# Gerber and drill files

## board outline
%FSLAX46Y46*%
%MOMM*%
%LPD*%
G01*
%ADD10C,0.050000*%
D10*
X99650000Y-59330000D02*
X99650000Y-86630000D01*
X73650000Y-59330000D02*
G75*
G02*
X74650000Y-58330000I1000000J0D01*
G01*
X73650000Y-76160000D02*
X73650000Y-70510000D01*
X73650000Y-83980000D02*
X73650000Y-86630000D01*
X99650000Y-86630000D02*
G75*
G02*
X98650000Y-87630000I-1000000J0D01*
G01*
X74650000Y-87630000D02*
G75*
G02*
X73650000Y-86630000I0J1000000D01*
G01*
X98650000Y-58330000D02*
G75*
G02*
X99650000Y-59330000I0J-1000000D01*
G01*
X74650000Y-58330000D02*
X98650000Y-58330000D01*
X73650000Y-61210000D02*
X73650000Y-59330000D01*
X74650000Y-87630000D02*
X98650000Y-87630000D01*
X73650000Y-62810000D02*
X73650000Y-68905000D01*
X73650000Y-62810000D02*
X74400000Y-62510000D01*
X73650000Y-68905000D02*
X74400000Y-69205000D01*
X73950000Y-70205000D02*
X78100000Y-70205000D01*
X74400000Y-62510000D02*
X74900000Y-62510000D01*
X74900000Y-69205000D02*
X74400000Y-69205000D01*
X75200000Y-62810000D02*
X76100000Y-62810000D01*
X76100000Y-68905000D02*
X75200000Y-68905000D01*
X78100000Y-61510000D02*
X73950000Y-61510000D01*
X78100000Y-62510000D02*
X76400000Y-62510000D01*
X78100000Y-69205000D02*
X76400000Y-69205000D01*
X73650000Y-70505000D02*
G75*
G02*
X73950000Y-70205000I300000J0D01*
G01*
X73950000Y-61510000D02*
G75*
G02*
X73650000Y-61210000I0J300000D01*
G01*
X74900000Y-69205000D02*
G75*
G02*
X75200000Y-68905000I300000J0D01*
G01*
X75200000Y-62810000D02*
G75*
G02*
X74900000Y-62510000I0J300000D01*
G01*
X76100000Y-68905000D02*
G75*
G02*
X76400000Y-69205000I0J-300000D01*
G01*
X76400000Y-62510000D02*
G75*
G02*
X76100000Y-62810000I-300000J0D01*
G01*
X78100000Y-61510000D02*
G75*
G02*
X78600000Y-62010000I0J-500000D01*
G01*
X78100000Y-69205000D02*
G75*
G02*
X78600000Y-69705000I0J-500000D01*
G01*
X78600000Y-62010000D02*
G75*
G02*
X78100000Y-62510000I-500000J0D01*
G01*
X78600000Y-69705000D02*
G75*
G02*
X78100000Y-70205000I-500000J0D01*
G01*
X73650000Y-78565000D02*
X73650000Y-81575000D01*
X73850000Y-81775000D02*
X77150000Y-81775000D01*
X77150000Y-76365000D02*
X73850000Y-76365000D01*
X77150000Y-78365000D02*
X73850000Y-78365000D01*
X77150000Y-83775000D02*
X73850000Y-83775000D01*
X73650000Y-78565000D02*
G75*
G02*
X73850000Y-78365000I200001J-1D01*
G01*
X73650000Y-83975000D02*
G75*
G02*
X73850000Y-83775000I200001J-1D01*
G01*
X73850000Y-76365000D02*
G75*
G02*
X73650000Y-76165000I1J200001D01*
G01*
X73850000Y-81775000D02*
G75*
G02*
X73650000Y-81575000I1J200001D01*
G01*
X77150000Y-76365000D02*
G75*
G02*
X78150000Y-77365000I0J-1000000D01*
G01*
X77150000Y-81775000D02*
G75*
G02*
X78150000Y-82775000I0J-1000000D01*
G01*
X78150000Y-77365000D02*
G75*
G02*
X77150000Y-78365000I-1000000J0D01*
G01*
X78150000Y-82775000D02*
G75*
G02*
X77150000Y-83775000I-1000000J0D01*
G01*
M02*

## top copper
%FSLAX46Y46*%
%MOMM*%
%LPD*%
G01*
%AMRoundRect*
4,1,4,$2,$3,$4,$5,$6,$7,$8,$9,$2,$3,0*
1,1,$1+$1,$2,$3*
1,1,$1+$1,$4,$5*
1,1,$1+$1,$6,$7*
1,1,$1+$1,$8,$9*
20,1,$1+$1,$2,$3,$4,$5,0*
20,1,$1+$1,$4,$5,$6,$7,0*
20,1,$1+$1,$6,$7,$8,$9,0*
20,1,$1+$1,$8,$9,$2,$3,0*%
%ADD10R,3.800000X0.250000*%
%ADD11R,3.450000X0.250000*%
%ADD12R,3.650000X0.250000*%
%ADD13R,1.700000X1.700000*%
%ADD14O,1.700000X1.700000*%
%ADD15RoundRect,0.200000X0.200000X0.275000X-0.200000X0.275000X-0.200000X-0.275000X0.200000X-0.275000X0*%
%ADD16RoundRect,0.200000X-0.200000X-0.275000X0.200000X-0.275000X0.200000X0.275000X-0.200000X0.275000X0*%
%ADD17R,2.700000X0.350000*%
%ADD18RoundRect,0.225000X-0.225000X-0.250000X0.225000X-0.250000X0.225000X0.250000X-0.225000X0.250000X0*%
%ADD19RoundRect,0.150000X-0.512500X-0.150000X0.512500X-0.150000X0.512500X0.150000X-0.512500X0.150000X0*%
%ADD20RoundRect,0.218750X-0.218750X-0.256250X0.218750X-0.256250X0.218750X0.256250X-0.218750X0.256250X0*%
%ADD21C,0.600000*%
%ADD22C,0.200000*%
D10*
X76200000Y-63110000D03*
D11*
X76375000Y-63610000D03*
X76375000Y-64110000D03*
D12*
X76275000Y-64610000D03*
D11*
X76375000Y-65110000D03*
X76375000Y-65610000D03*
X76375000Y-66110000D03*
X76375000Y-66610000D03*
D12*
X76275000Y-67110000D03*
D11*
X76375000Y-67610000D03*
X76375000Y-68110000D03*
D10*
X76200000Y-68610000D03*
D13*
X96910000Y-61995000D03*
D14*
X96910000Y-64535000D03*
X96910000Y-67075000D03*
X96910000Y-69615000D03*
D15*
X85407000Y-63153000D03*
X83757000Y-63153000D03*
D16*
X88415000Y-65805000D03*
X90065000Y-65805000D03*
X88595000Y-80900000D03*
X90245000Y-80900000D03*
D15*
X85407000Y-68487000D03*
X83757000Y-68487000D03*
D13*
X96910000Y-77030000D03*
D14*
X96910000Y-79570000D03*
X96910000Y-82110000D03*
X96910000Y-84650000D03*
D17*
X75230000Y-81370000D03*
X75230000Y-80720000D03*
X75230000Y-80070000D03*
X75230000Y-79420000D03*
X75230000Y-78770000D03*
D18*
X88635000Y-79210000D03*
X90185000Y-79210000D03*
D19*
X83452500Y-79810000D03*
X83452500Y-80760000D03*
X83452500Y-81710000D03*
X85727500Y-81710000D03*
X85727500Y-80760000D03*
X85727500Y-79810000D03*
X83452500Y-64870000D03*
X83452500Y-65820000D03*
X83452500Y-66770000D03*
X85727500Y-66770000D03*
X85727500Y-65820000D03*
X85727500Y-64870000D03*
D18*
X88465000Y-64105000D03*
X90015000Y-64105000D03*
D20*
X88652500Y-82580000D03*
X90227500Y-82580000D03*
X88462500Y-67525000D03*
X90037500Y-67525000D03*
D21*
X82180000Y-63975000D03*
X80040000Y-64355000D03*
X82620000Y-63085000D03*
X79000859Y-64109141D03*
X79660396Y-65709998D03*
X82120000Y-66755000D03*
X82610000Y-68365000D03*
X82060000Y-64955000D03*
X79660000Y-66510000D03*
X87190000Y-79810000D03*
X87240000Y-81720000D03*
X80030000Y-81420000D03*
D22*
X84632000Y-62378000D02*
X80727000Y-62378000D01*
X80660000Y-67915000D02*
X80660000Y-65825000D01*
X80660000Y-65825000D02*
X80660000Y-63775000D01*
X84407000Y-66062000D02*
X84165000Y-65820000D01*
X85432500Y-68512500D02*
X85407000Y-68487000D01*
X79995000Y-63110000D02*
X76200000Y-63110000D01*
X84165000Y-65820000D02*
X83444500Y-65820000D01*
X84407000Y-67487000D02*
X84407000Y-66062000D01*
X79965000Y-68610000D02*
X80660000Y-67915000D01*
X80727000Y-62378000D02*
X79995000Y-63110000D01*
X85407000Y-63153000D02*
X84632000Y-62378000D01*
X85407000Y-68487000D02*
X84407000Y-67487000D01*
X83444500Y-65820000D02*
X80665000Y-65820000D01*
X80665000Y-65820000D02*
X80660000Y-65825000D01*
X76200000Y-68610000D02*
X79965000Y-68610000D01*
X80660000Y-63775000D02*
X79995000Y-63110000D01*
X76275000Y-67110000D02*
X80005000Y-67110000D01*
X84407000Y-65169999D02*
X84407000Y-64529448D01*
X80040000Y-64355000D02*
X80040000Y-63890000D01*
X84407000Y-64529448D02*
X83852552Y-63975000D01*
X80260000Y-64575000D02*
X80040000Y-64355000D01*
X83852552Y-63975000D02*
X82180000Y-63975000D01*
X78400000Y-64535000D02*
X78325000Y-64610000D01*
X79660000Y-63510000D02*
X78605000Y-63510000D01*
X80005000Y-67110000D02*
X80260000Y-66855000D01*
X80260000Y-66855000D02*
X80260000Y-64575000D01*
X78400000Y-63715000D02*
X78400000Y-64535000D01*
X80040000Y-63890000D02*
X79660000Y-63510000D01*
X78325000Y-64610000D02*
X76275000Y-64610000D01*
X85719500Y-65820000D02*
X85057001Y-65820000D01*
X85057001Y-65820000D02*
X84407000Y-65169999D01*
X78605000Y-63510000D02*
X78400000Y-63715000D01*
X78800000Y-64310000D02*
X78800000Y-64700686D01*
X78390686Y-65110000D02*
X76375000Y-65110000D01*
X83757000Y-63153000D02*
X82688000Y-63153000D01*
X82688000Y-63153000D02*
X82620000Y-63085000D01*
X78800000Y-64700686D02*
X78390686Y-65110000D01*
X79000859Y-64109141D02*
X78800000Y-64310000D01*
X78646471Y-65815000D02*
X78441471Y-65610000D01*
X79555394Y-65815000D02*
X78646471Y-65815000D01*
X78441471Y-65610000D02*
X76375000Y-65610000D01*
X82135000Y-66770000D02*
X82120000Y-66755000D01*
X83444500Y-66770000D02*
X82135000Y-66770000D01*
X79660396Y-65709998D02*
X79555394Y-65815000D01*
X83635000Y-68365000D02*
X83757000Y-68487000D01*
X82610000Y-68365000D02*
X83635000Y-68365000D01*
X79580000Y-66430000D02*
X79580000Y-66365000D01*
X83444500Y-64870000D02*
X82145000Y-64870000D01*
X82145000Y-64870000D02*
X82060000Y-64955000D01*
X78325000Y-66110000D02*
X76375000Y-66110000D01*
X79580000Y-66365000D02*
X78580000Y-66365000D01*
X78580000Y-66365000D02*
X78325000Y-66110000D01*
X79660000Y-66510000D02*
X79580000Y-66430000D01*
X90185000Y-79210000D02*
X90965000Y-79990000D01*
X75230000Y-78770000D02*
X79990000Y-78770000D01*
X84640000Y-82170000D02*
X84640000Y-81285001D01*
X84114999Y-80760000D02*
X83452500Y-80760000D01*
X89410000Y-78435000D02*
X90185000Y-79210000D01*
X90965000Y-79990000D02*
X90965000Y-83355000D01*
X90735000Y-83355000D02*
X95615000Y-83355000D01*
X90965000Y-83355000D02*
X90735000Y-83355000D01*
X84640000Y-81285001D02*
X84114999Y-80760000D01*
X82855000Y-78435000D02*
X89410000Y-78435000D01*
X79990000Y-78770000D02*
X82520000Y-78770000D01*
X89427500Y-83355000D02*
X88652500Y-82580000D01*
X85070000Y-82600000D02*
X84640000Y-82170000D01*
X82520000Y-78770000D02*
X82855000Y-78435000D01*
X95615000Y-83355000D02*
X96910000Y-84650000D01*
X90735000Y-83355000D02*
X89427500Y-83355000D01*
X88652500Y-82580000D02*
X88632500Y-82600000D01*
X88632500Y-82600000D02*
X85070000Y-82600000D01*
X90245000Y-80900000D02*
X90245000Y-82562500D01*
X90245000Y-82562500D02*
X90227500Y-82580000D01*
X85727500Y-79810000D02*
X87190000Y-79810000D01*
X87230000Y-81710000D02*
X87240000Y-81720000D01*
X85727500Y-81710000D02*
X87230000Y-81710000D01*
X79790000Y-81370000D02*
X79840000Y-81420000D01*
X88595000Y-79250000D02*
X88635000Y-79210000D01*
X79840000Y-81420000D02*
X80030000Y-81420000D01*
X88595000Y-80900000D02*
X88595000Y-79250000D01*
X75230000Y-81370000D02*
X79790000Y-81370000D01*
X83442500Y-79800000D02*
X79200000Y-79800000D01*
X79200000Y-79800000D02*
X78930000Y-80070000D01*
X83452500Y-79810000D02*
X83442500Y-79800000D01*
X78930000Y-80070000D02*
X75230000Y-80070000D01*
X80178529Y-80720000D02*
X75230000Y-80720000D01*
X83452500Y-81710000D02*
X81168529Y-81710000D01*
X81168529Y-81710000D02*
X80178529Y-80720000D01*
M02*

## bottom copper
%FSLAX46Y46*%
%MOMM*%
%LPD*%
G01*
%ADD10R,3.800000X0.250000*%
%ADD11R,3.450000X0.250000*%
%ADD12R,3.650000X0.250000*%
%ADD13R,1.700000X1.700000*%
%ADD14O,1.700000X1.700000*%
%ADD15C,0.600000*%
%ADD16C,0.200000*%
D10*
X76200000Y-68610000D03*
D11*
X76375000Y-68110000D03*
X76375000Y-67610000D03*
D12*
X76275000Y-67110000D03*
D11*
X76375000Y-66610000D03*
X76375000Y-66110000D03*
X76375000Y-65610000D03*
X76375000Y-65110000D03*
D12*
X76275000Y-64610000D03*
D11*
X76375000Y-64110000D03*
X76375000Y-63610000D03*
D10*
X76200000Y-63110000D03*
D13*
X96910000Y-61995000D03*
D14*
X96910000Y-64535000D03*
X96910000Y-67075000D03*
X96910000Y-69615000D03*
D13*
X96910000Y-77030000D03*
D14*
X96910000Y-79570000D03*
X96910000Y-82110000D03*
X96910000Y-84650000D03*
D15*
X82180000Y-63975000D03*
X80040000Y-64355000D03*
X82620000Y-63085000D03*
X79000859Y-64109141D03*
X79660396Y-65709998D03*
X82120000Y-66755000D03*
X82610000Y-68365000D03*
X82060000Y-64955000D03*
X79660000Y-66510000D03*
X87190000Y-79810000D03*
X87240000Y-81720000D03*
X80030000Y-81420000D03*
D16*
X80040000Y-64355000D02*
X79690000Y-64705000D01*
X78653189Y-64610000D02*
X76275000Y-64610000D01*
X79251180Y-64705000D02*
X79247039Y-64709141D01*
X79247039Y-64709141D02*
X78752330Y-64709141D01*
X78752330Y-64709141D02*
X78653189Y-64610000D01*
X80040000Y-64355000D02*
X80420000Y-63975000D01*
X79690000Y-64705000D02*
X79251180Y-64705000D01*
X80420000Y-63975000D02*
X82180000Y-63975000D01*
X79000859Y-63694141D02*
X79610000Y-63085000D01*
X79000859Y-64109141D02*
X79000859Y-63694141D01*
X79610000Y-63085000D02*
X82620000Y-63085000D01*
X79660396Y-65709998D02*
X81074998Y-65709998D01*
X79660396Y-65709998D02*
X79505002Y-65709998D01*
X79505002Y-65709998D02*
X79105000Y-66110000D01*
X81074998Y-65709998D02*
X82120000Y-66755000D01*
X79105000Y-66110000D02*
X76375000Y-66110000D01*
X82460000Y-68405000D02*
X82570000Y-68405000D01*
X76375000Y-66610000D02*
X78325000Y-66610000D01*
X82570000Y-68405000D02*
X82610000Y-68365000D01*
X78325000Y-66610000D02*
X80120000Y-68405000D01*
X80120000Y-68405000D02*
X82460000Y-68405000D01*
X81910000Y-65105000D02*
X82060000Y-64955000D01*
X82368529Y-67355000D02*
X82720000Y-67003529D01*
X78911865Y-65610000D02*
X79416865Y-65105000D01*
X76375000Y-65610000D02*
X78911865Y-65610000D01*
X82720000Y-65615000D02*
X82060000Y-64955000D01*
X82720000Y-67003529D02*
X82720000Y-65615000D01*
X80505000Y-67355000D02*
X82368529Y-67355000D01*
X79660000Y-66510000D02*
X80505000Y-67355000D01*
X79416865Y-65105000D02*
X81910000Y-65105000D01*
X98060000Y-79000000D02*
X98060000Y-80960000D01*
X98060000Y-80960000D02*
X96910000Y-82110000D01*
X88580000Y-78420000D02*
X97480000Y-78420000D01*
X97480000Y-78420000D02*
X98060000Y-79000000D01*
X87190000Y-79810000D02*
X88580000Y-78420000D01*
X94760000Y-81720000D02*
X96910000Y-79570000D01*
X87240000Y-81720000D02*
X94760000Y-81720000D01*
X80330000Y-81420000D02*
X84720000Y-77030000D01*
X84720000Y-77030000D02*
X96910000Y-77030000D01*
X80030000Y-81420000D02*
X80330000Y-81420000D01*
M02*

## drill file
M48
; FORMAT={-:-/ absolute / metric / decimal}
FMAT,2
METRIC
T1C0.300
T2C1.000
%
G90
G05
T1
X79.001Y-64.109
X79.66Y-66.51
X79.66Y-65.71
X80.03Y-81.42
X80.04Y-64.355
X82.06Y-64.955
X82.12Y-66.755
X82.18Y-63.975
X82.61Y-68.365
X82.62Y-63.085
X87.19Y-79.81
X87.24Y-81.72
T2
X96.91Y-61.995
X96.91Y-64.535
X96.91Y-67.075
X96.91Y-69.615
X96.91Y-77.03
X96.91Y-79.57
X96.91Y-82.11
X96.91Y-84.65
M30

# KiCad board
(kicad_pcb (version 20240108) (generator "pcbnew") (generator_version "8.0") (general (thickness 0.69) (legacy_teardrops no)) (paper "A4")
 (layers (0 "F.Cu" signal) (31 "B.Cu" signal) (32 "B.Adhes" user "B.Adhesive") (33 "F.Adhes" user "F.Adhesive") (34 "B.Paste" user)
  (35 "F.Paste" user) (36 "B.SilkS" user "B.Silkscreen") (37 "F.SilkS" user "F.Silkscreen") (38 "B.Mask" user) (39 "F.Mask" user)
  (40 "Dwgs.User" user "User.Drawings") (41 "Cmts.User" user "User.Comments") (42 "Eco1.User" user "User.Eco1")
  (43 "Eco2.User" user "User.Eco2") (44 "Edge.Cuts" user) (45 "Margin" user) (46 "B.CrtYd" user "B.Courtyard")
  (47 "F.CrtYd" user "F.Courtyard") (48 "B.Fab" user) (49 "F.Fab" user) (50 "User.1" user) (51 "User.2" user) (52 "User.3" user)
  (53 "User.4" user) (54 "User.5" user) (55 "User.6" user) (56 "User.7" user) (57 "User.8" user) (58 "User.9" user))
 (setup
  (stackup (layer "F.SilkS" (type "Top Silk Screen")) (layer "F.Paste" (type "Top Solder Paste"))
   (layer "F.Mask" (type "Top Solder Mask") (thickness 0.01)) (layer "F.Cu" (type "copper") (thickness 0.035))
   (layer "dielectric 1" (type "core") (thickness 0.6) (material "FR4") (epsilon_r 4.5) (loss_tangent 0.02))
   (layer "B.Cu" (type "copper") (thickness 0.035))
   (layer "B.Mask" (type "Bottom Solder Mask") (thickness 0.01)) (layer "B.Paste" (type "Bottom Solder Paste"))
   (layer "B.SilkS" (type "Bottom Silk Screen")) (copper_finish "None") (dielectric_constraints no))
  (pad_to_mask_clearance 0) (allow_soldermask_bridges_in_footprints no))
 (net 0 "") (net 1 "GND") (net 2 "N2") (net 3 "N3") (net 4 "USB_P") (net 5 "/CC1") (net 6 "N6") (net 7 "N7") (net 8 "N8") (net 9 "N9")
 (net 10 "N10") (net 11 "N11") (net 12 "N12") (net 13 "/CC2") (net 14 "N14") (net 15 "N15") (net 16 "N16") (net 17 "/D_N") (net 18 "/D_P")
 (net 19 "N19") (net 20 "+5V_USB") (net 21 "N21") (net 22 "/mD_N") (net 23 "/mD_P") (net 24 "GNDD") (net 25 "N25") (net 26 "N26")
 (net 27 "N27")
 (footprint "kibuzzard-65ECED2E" (layer "F.Cu") (at 93.23 82.17)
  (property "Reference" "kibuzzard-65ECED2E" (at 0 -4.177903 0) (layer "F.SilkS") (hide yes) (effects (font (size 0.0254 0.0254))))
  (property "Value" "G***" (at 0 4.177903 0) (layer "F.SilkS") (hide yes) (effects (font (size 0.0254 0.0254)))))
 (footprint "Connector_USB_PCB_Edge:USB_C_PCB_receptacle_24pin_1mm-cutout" (layer "F.Cu") (at 76.2 65.86)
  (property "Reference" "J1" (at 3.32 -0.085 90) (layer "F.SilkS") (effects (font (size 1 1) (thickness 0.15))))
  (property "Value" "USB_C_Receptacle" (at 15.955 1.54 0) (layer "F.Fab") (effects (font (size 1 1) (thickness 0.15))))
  (fp_line (start -2.55 -3.05) (end -2.55 3.045) (stroke (width 0.05) (type default)) (layer "Edge.Cuts"))
  (fp_line (start -2.55 -3.05) (end -1.8 -3.35) (stroke (width 0.05) (type default)) (layer "Edge.Cuts"))
  (fp_line (start -2.55 3.045) (end -1.8 3.345) (stroke (width 0.05) (type default)) (layer "Edge.Cuts"))
  (fp_line (start -2.25 4.345) (end 1.9 4.345) (stroke (width 0.05) (type default)) (layer "Edge.Cuts"))
  (fp_line (start -1.8 -3.35) (end -1.3 -3.35) (stroke (width 0.05) (type default)) (layer "Edge.Cuts"))
  (fp_line (start -1.3 3.345) (end -1.8 3.345) (stroke (width 0.05) (type default)) (layer "Edge.Cuts"))
  (fp_line (start -1 -3.05) (end -0.1 -3.05) (stroke (width 0.05) (type default)) (layer "Edge.Cuts"))
  (fp_line (start -0.1 3.045) (end -1 3.045) (stroke (width 0.05) (type default)) (layer "Edge.Cuts"))
  (fp_line (start 1.9 -4.35) (end -2.25 -4.35) (stroke (width 0.05) (type default)) (layer "Edge.Cuts"))
  (fp_line (start 1.9 -3.35) (end 0.2 -3.35) (stroke (width 0.05) (type default)) (layer "Edge.Cuts"))
  (fp_line (start 1.9 3.345) (end 0.2 3.345) (stroke (width 0.05) (type default)) (layer "Edge.Cuts"))
  (fp_arc (start -2.55 4.645) (mid -2.462132 4.432868) (end -2.25 4.345) (stroke (width 0.05) (type default)) (layer "Edge.Cuts"))
  (fp_arc (start -2.25 -4.35) (mid -2.462132 -4.437868) (end -2.55 -4.65) (stroke (width 0.05) (type default)) (layer "Edge.Cuts"))
  (fp_arc (start -1.3 3.345) (mid -1.212132 3.132868) (end -1 3.045) (stroke (width 0.05) (type default)) (layer "Edge.Cuts"))
  (fp_arc (start -1 -3.05) (mid -1.212132 -3.137868) (end -1.3 -3.35) (stroke (width 0.05) (type default)) (layer "Edge.Cuts"))
  (fp_arc (start -0.1 3.045) (mid 0.112132 3.132868) (end 0.2 3.345) (stroke (width 0.05) (type default)) (layer "Edge.Cuts"))
  (fp_arc (start 0.2 -3.35) (mid 0.112132 -3.137868) (end -0.1 -3.05) (stroke (width 0.05) (type default)) (layer "Edge.Cuts"))
  (fp_arc (start 1.9 -4.35) (mid 2.253553 -4.203553) (end 2.4 -3.85) (stroke (width 0.05) (type default)) (layer "Edge.Cuts"))
  (fp_arc (start 1.9 3.345) (mid 2.253553 3.491447) (end 2.4 3.845) (stroke (width 0.05) (type default)) (layer "Edge.Cuts"))
  (fp_arc (start 2.4 -3.85) (mid 2.253553 -3.496447) (end 1.9 -3.35) (stroke (width 0.05) (type default)) (layer "Edge.Cuts"))
  (fp_arc (start 2.4 3.845) (mid 2.253553 4.198553) (end 1.9 4.345) (stroke (width 0.05) (type default)) (layer "Edge.Cuts"))
  (pad "A1" smd rect (at 0 -2.75 270) (size 0.25 3.8) (layers "F.Cu" "F.Paste" "F.Mask") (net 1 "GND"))
  (pad "A2" smd rect (at 0.175 -2.25 270) (size 0.25 3.45) (layers "F.Cu" "F.Paste" "F.Mask") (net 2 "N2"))
  (pad "A3" smd rect (at 0.175 -1.75 270) (size 0.25 3.45) (layers "F.Cu" "F.Paste" "F.Mask") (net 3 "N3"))
  (pad "A4" smd rect (at 0.075 -1.25 270) (size 0.25 3.65) (layers "F.Cu" "F.Paste" "F.Mask") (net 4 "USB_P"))
  (pad "A5" smd rect (at 0.175 -0.75 270) (size 0.25 3.45) (layers "F.Cu" "F.Paste" "F.Mask") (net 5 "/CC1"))
  (pad "A6" smd rect (at 0.175 -0.25 270) (size 0.25 3.45) (layers "F.Cu" "F.Paste" "F.Mask") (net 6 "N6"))
  (pad "A7" smd rect (at 0.175 0.25 270) (size 0.25 3.45) (layers "F.Cu" "F.Paste" "F.Mask") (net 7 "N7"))
  (pad "A8" smd rect (at 0.175 0.75 270) (size 0.25 3.45) (layers "F.Cu" "F.Paste" "F.Mask") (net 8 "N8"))
  (pad "A9" smd rect (at 0.075 1.25 270) (size 0.25 3.65) (layers "F.Cu" "F.Paste" "F.Mask") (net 4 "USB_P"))
  (pad "A10" smd rect (at 0.175 1.75 270) (size 0.25 3.45) (layers "F.Cu" "F.Paste" "F.Mask") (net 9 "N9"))
  (pad "A11" smd rect (at 0.175 2.25 270) (size 0.25 3.45) (layers "F.Cu" "F.Paste" "F.Mask") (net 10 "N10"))
  (pad "A12" smd rect (at 0 2.75 270) (size 0.25 3.8) (layers "F.Cu" "F.Paste" "F.Mask") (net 1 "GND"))
  (pad "B1" smd rect (at 0 2.75 270) (size 0.25 3.8) (layers "B.Cu" "B.Paste" "B.Mask") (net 1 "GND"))
  (pad "B2" smd rect (at 0.175 2.25 270) (size 0.25 3.45) (layers "B.Cu" "B.Paste" "B.Mask") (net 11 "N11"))
  (pad "B3" smd rect (at 0.175 1.75 270) (size 0.25 3.45) (layers "B.Cu" "B.Paste" "B.Mask") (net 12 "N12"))
  (pad "B4" smd rect (at 0.075 1.25 270) (size 0.25 3.65) (layers "B.Cu" "B.Paste" "B.Mask") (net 4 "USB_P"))
  (pad "B5" smd rect (at 0.175 0.75 270) (size 0.25 3.45) (layers "B.Cu" "B.Paste" "B.Mask") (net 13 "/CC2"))
  (pad "B6" smd rect (at 0.175 0.25 270) (size 0.25 3.45) (layers "B.Cu" "B.Paste" "B.Mask") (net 6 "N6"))
  (pad "B7" smd rect (at 0.175 -0.25 270) (size 0.25 3.45) (layers "B.Cu" "B.Paste" "B.Mask") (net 7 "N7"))
  (pad "B8" smd rect (at 0.175 -0.75 270) (size 0.25 3.45) (layers "B.Cu" "B.Paste" "B.Mask") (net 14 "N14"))
  (pad "B9" smd rect (at 0.075 -1.25 270) (size 0.25 3.65) (layers "B.Cu" "B.Paste" "B.Mask") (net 4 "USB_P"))
  (pad "B10" smd rect (at 0.175 -1.75 270) (size 0.25 3.45) (layers "B.Cu" "B.Paste" "B.Mask") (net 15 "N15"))
  (pad "B11" smd rect (at 0.175 -2.25 270) (size 0.25 3.45) (layers "B.Cu" "B.Paste" "B.Mask") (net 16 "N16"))
  (pad "B12" smd rect (at 0 -2.75 270) (size 0.25 3.8) (layers "B.Cu" "B.Paste" "B.Mask") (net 1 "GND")))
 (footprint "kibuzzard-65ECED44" (layer "F.Cu") (at 92.15 84.75)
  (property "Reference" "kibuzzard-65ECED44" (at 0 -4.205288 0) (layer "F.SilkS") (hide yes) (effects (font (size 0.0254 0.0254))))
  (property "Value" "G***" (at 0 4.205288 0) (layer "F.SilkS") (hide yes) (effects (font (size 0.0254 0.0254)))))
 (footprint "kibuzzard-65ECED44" (layer "F.Cu") (at 92.12 69.685)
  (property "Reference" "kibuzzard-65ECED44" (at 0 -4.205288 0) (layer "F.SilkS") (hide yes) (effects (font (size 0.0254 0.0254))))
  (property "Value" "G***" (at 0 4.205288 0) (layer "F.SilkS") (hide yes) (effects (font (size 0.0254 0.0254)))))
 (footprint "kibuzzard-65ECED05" (layer "F.Cu") (at 92.37 61.865)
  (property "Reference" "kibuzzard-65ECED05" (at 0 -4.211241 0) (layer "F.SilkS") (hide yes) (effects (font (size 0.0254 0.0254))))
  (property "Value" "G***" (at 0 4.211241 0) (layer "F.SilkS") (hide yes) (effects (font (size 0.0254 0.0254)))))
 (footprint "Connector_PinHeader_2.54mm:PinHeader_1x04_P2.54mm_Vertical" (layer "F.Cu") (at 96.91 61.995)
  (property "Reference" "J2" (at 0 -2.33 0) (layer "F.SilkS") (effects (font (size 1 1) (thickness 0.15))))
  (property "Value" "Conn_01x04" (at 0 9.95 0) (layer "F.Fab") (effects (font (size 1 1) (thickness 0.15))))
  (pad "1" thru_hole rect (at 0 0) (size 1.7 1.7) (drill 1) (layers "*.Cu" "*.Mask") (remove_unused_layers no) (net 4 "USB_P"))
  (pad "2" thru_hole oval (at 0 2.54) (size 1.7 1.7) (drill 1) (layers "*.Cu" "*.Mask") (remove_unused_layers no) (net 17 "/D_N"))
  (pad "3" thru_hole oval (at 0 5.08) (size 1.7 1.7) (drill 1) (layers "*.Cu" "*.Mask") (remove_unused_layers no) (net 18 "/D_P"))
  (pad "4" thru_hole oval (at 0 7.62) (size 1.7 1.7) (drill 1) (layers "*.Cu" "*.Mask") (remove_unused_layers no) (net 1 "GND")))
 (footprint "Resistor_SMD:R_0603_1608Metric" (layer "F.Cu") (at 84.582 63.153 180)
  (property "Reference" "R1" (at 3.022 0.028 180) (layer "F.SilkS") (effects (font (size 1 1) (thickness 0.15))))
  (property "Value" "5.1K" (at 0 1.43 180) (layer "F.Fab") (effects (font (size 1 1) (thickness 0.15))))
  (pad "1" smd roundrect (at -0.825 0 180) (size 0.8 0.95) (layers "F.Cu" "F.Paste" "F.Mask") (roundrect_rratio 0.25) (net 1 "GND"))
  (pad "2" smd roundrect (at 0.825 0 180) (size 0.8 0.95) (layers "F.Cu" "F.Paste" "F.Mask") (roundrect_rratio 0.25) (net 5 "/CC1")))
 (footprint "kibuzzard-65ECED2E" (layer "F.Cu") (at 93.2 67.105)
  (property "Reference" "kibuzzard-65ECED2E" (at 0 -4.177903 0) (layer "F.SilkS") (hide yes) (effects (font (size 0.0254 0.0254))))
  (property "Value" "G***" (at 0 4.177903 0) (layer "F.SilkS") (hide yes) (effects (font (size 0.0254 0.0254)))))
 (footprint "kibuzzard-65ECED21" (layer "F.Cu") (at 93.14 79.59)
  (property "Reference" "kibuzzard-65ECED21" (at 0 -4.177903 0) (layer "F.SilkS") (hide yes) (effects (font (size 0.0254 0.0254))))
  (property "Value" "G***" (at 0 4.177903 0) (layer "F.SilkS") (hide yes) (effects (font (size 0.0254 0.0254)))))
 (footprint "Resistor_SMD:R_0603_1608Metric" (layer "F.Cu") (at 89.24 65.805)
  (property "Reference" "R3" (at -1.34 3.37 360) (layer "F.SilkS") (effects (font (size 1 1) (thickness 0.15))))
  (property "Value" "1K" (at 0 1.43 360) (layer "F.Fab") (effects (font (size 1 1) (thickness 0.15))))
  (pad "1" smd roundrect (at -0.825 0) (size 0.8 0.95) (layers "F.Cu" "F.Paste" "F.Mask") (roundrect_rratio 0.25) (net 4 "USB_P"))
  (pad "2" smd roundrect (at 0.825 0) (size 0.8 0.95) (layers "F.Cu" "F.Paste" "F.Mask") (roundrect_rratio 0.25) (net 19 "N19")))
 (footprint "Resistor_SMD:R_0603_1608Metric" (layer "F.Cu") (at 89.42 80.9)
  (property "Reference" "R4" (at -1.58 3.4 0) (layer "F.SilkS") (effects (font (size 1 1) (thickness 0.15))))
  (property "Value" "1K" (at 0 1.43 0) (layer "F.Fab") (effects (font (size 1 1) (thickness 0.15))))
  (pad "1" smd roundrect (at -0.825 0) (size 0.8 0.95) (layers "F.Cu" "F.Paste" "F.Mask") (roundrect_rratio 0.25) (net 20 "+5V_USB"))
  (pad "2" smd roundrect (at 0.825 0) (size 0.8 0.95) (layers "F.Cu" "F.Paste" "F.Mask") (roundrect_rratio 0.25) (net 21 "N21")))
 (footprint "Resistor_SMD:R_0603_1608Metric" (layer "F.Cu") (at 84.582 68.487 180)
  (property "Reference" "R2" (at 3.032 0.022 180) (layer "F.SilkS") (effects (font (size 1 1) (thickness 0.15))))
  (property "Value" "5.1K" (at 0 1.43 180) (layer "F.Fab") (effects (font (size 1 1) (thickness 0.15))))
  (pad "1" smd roundrect (at -0.825 0 180) (size 0.8 0.95) (layers "F.Cu" "F.Paste" "F.Mask") (roundrect_rratio 0.25) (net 1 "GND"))
  (pad "2" smd roundrect (at 0.825 0 180) (size 0.8 0.95) (layers "F.Cu" "F.Paste" "F.Mask") (roundrect_rratio 0.25) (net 13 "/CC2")))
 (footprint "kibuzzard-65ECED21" (layer "F.Cu") (at 93.11 64.525)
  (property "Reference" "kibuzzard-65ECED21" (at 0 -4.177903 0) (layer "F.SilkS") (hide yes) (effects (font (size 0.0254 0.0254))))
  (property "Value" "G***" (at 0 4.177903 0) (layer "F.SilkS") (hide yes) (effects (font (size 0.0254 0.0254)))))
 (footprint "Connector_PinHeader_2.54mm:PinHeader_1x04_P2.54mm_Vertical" (layer "F.Cu") (at 96.91 77.03)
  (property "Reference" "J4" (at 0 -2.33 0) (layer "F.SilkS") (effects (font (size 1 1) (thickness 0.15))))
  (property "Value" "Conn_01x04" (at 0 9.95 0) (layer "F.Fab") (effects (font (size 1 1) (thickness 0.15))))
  (pad "1" thru_hole rect (at 0 0) (size 1.7 1.7) (drill 1) (layers "*.Cu" "*.Mask") (remove_unused_layers no) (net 20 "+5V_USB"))
  (pad "2" thru_hole oval (at 0 2.54) (size 1.7 1.7) (drill 1) (layers "*.Cu" "*.Mask") (remove_unused_layers no) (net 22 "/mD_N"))
  (pad "3" thru_hole oval (at 0 5.08) (size 1.7 1.7) (drill 1) (layers "*.Cu" "*.Mask") (remove_unused_layers no) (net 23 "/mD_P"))
  (pad "4" thru_hole oval (at 0 7.62) (size 1.7 1.7) (drill 1) (layers "*.Cu" "*.Mask") (remove_unused_layers no) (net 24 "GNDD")))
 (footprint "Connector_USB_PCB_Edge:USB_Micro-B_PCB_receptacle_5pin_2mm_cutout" (layer "F.Cu") (at 75.23 80.07)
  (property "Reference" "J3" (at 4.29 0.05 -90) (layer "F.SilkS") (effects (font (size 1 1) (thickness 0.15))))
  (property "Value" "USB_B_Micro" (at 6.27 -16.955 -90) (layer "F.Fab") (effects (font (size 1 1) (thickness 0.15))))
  (fp_line (start -1.58 -1.505) (end -1.58 1.505) (stroke (width 0.05) (type default)) (layer "Edge.Cuts"))
  (fp_line (start -1.38 1.705) (end 1.92 1.705) (stroke (width 0.05) (type default)) (layer "Edge.Cuts"))
  (fp_line (start 1.92 -3.705) (end -1.38 -3.705) (stroke (width 0.05) (type default)) (layer "Edge.Cuts"))
  (fp_line (start 1.92 -1.705) (end -1.38 -1.705) (stroke (width 0.05) (type default)) (layer "Edge.Cuts"))
  (fp_line (start 1.92 3.705) (end -1.38 3.705) (stroke (width 0.05) (type default)) (layer "Edge.Cuts"))
  (fp_arc (start -1.58 -1.505) (mid -1.521421 -1.646421) (end -1.38 -1.705) (stroke (width 0.05) (type default)) (layer "Edge.Cuts"))
  (fp_arc (start -1.58 3.905) (mid -1.521421 3.763579) (end -1.38 3.705) (stroke (width 0.05) (type default)) (layer "Edge.Cuts"))
  (fp_arc (start -1.38 -3.705) (mid -1.521421 -3.763579) (end -1.58 -3.905) (stroke (width 0.05) (type default)) (layer "Edge.Cuts"))
  (fp_arc (start -1.38 1.705) (mid -1.521421 1.646421) (end -1.58 1.505) (stroke (width 0.05) (type default)) (layer "Edge.Cuts"))
  (fp_arc (start 1.92 -3.705) (mid 2.627107 -3.412107) (end 2.92 -2.705) (stroke (width 0.05) (type default)) (layer "Edge.Cuts"))
  (fp_arc (start 1.92 1.705) (mid 2.627107 1.997893) (end 2.92 2.705) (stroke (width 0.05) (type default)) (layer "Edge.Cuts"))
  (fp_arc (start 2.92 -2.705) (mid 2.627107 -1.997893) (end 1.92 -1.705) (stroke (width 0.05) (type default)) (layer "Edge.Cuts"))
  (fp_arc (start 2.92 2.705) (mid 2.627107 3.412107) (end 1.92 3.705) (stroke (width 0.05) (type default)) (layer "Edge.Cuts"))
  (pad "1" smd rect (at 0 1.3 90) (size 0.35 2.7) (layers "F.Cu" "F.Paste" "F.Mask") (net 20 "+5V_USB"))
  (pad "2" smd rect (at 0 0.65 90) (size 0.35 2.7) (layers "F.Cu" "F.Paste" "F.Mask") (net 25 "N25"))
  (pad "3" smd rect (at 0 0 90) (size 0.35 2.7) (layers "F.Cu" "F.Paste" "F.Mask") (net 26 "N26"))
  (pad "4" smd rect (at 0 -0.65 90) (size 0.35 2.7) (layers "F.Cu" "F.Paste" "F.Mask") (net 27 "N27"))
  (pad "5" smd rect (at 0 -1.3 90) (size 0.35 2.7) (layers "F.Cu" "F.Paste" "F.Mask") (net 24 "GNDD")))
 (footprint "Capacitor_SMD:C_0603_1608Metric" (layer "F.Cu") (at 89.41 79.21)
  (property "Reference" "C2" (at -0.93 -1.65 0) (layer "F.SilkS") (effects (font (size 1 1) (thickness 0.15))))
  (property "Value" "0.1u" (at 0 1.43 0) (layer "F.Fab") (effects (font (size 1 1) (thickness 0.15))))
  (pad "1" smd roundrect (at -0.775 0) (size 0.9 0.95) (layers "F.Cu" "F.Paste" "F.Mask") (roundrect_rratio 0.25) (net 20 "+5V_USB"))
  (pad "2" smd roundrect (at 0.775 0) (size 0.9 0.95) (layers "F.Cu" "F.Paste" "F.Mask") (roundrect_rratio 0.25) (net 24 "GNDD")))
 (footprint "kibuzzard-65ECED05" (layer "F.Cu") (at 92.4 76.93)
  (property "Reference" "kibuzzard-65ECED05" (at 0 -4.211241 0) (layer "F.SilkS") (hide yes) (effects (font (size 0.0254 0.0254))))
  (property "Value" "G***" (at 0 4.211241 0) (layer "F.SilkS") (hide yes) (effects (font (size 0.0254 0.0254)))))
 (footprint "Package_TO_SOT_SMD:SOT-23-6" (layer "F.Cu") (at 84.59 80.76)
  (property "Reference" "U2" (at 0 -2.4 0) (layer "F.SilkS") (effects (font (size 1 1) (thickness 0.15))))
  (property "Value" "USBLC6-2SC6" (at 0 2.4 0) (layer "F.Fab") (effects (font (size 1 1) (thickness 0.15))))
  (pad "1" smd roundrect (at -1.1375 -0.95) (size 1.325 0.6) (layers "F.Cu" "F.Paste" "F.Mask") (roundrect_rratio 0.25) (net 26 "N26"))
  (pad "2" smd roundrect (at -1.1375 0) (size 1.325 0.6) (layers "F.Cu" "F.Paste" "F.Mask") (roundrect_rratio 0.25) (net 24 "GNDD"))
  (pad "3" smd roundrect (at -1.1375 0.95) (size 1.325 0.6) (layers "F.Cu" "F.Paste" "F.Mask") (roundrect_rratio 0.25) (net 25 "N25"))
  (pad "4" smd roundrect (at 1.1375 0.95) (size 1.325 0.6) (layers "F.Cu" "F.Paste" "F.Mask") (roundrect_rratio 0.25) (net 22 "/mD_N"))
  (pad "5" smd roundrect (at 1.1375 0) (size 1.325 0.6) (layers "F.Cu" "F.Paste" "F.Mask") (roundrect_rratio 0.25) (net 20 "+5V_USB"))
  (pad "6" smd roundrect (at 1.1375 -0.95) (size 1.325 0.6) (layers "F.Cu" "F.Paste" "F.Mask") (roundrect_rratio 0.25) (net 23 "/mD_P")))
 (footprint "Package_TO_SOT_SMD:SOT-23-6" (layer "F.Cu") (at 84.59 65.82)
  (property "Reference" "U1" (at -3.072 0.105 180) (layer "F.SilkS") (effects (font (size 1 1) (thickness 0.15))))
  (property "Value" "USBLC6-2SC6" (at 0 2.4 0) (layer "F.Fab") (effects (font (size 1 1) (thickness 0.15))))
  (pad "1" smd roundrect (at -1.1375 -0.95) (size 1.325 0.6) (layers "F.Cu" "F.Paste" "F.Mask") (roundrect_rratio 0.25) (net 7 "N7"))
  (pad "2" smd roundrect (at -1.1375 0) (size 1.325 0.6) (layers "F.Cu" "F.Paste" "F.Mask") (roundrect_rratio 0.25) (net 1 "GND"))
  (pad "3" smd roundrect (at -1.1375 0.95) (size 1.325 0.6) (layers "F.Cu" "F.Paste" "F.Mask") (roundrect_rratio 0.25) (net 6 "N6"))
  (pad "4" smd roundrect (at 1.1375 0.95) (size 1.325 0.6) (layers "F.Cu" "F.Paste" "F.Mask") (roundrect_rratio 0.25) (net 18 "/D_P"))
  (pad "5" smd roundrect (at 1.1375 0) (size 1.325 0.6) (layers "F.Cu" "F.Paste" "F.Mask") (roundrect_rratio 0.25) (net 4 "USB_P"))
  (pad "6" smd roundrect (at 1.1375 -0.95) (size 1.325 0.6) (layers "F.Cu" "F.Paste" "F.Mask") (roundrect_rratio 0.25) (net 17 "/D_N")))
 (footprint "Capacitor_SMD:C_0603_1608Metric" (layer "F.Cu") (at 89.24 64.105)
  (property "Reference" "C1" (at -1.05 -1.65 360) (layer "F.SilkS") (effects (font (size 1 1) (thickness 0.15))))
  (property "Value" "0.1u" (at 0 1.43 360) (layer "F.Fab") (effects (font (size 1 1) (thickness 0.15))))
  (pad "1" smd roundrect (at -0.775 0) (size 0.9 0.95) (layers "F.Cu" "F.Paste" "F.Mask") (roundrect_rratio 0.25) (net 4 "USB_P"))
  (pad "2" smd roundrect (at 0.775 0) (size 0.9 0.95) (layers "F.Cu" "F.Paste" "F.Mask") (roundrect_rratio 0.25) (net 1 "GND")))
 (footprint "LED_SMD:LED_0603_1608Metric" (layer "F.Cu") (at 89.44 82.58)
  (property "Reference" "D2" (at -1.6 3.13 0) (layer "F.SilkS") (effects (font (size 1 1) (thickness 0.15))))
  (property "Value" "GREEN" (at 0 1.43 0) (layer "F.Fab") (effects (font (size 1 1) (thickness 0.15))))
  (pad "1" smd roundrect (at -0.7875 0) (size 0.875 0.95) (layers "F.Cu" "F.Paste" "F.Mask") (roundrect_rratio 0.25) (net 24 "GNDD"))
  (pad "2" smd roundrect (at 0.7875 0) (size 0.875 0.95) (layers "F.Cu" "F.Paste" "F.Mask") (roundrect_rratio 0.25) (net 21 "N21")))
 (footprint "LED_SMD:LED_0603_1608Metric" (layer "F.Cu") (at 89.25 67.525)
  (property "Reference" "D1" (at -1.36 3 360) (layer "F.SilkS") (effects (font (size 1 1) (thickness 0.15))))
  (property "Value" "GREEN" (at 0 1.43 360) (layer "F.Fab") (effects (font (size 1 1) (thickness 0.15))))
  (pad "1" smd roundrect (at -0.7875 0) (size 0.875 0.95) (layers "F.Cu" "F.Paste" "F.Mask") (roundrect_rratio 0.25) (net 1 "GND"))
  (pad "2" smd roundrect (at 0.7875 0) (size 0.875 0.95) (layers "F.Cu" "F.Paste" "F.Mask") (roundrect_rratio 0.25) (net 19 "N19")))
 (gr_line (start 99.65 59.33) (end 99.65 86.63) (stroke (width 0.05) (type default)) (layer "Edge.Cuts"))
 (gr_arc (start 73.65 59.33) (mid 73.942893 58.622893) (end 74.65 58.33) (stroke (width 0.05) (type default)) (layer "Edge.Cuts"))
 (gr_line (start 73.65 76.16) (end 73.65 70.51) (stroke (width 0.05) (type default)) (layer "Edge.Cuts"))
 (gr_line (start 73.65 83.98) (end 73.65 86.63) (stroke (width 0.05) (type default)) (layer "Edge.Cuts"))
 (gr_arc (start 99.65 86.63) (mid 99.357107 87.337107) (end 98.65 87.63) (stroke (width 0.05) (type default)) (layer "Edge.Cuts"))
 (gr_arc (start 74.65 87.63) (mid 73.942893 87.337107) (end 73.65 86.63) (stroke (width 0.05) (type default)) (layer "Edge.Cuts"))
 (gr_arc (start 98.65 58.33) (mid 99.357107 58.622893) (end 99.65 59.33) (stroke (width 0.05) (type default)) (layer "Edge.Cuts"))
 (gr_line (start 74.65 58.33) (end 98.65 58.33) (stroke (width 0.05) (type default)) (layer "Edge.Cuts"))
 (gr_line (start 73.65 61.21) (end 73.65 59.33) (stroke (width 0.05) (type default)) (layer "Edge.Cuts"))
 (gr_line (start 74.65 87.63) (end 98.65 87.63) (stroke (width 0.05) (type default)) (layer "Edge.Cuts"))
 (segment (start 84.632 62.378) (end 80.727 62.378) (width 0.2) (layer "F.Cu") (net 1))
 (segment (start 80.66 67.915) (end 80.66 65.825) (width 0.2) (layer "F.Cu") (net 1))
 (segment (start 80.66 65.825) (end 80.66 63.775) (width 0.2) (layer "F.Cu") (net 1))
 (segment (start 84.407 66.062) (end 84.165 65.82) (width 0.2) (layer "F.Cu") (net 1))
 (segment (start 85.4325 68.5125) (end 85.407 68.487) (width 0.2) (layer "F.Cu") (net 1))
 (segment (start 79.995 63.11) (end 76.2 63.11) (width 0.2) (layer "F.Cu") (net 1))
 (segment (start 84.165 65.82) (end 83.4445 65.82) (width 0.2) (layer "F.Cu") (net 1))
 (segment (start 84.407 67.487) (end 84.407 66.062) (width 0.2) (layer "F.Cu") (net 1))
 (segment (start 79.965 68.61) (end 80.66 67.915) (width 0.2) (layer "F.Cu") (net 1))
 (segment (start 80.727 62.378) (end 79.995 63.11) (width 0.2) (layer "F.Cu") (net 1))
 (segment (start 85.407 63.153) (end 84.632 62.378) (width 0.2) (layer "F.Cu") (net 1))
 (segment (start 85.407 68.487) (end 84.407 67.487) (width 0.2) (layer "F.Cu") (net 1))
 (segment (start 83.4445 65.82) (end 80.665 65.82) (width 0.2) (layer "F.Cu") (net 1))
 (segment (start 80.665 65.82) (end 80.66 65.825) (width 0.2) (layer "F.Cu") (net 1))
 (segment (start 76.2 68.61) (end 79.965 68.61) (width 0.2) (layer "F.Cu") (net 1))
 (segment (start 80.66 63.775) (end 79.995 63.11) (width 0.2) (layer "F.Cu") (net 1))
 (segment (start 76.275 67.11) (end 80.005 67.11) (width 0.2) (layer "F.Cu") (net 4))
 (segment (start 84.407 65.169999) (end 84.407 64.529448) (width 0.2) (layer "F.Cu") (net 4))
 (segment (start 80.04 64.355) (end 80.04 63.89) (width 0.2) (layer "F.Cu") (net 4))
 (segment (start 84.407 64.529448) (end 83.852552 63.975) (width 0.2) (layer "F.Cu") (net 4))
 (segment (start 80.26 64.575) (end 80.04 64.355) (width 0.2) (layer "F.Cu") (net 4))
 (segment (start 83.852552 63.975) (end 82.18 63.975) (width 0.2) (layer "F.Cu") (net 4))
 (segment (start 78.4 64.535) (end 78.325 64.61) (width 0.2) (layer "F.Cu") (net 4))
 (segment (start 79.66 63.51) (end 78.605 63.51) (width 0.2) (layer "F.Cu") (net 4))
 (segment (start 80.005 67.11) (end 80.26 66.855) (width 0.2) (layer "F.Cu") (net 4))
 (segment (start 80.26 66.855) (end 80.26 64.575) (width 0.2) (layer "F.Cu") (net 4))
 (segment (start 78.4 63.715) (end 78.4 64.535) (width 0.2) (layer "F.Cu") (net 4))
 (segment (start 80.04 63.89) (end 79.66 63.51) (width 0.2) (layer "F.Cu") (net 4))
 (segment (start 78.325 64.61) (end 76.275 64.61) (width 0.2) (layer "F.Cu") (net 4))
 (segment (start 85.7195 65.82) (end 85.057001 65.82) (width 0.2) (layer "F.Cu") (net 4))
 (segment (start 85.057001 65.82) (end 84.407 65.169999) (width 0.2) (layer "F.Cu") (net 4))
 (segment (start 78.605 63.51) (end 78.4 63.715) (width 0.2) (layer "F.Cu") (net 4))
 (via (at 82.18 63.975) (size 0.6) (drill 0.3) (layers "F.Cu" "B.Cu") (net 4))
 (via (at 80.04 64.355) (size 0.6) (drill 0.3) (layers "F.Cu" "B.Cu") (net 4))
 (segment (start 80.04 64.355) (end 79.69 64.705) (width 0.2) (layer "B.Cu") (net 4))
 (segment (start 78.653189 64.61) (end 76.275 64.61) (width 0.2) (layer "B.Cu") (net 4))
 (segment (start 79.25118 64.705) (end 79.247039 64.709141) (width 0.2) (layer "B.Cu") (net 4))
 (segment (start 79.247039 64.709141) (end 78.75233 64.709141) (width 0.2) (layer "B.Cu") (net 4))
 (segment (start 78.75233 64.709141) (end 78.653189 64.61) (width 0.2) (layer "B.Cu") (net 4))
 (segment (start 80.04 64.355) (end 80.42 63.975) (width 0.2) (layer "B.Cu") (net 4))
 (segment (start 79.69 64.705) (end 79.25118 64.705) (width 0.2) (layer "B.Cu") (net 4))
 (segment (start 80.42 63.975) (end 82.18 63.975) (width 0.2) (layer "B.Cu") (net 4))
 (segment (start 78.8 64.31) (end 78.8 64.700686) (width 0.2) (layer "F.Cu") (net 5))
 (segment (start 78.390686 65.11) (end 76.375 65.11) (width 0.2) (layer "F.Cu") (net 5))
 (segment (start 83.757 63.153) (end 82.688 63.153) (width 0.2) (layer "F.Cu") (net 5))
 (segment (start 82.688 63.153) (end 82.62 63.085) (width 0.2) (layer "F.Cu") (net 5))
 (segment (start 78.8 64.700686) (end 78.390686 65.11) (width 0.2) (layer "F.Cu") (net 5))
 (segment (start 79.000859 64.109141) (end 78.8 64.31) (width 0.2) (layer "F.Cu") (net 5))
 (via (at 82.62 63.085) (size 0.6) (drill 0.3) (layers "F.Cu" "B.Cu") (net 5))
 (via (at 79.000859 64.109141) (size 0.6) (drill 0.3) (layers "F.Cu" "B.Cu") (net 5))
 (segment (start 79.000859 63.694141) (end 79.61 63.085) (width 0.2) (layer "B.Cu") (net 5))
 (segment (start 79.000859 64.109141) (end 79.000859 63.694141) (width 0.2) (layer "B.Cu") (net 5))
 (segment (start 79.61 63.085) (end 82.62 63.085) (width 0.2) (layer "B.Cu") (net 5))
 (segment (start 78.646471 65.815) (end 78.441471 65.61) (width 0.2) (layer "F.Cu") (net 6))
 (segment (start 79.555394 65.815) (end 78.646471 65.815) (width 0.2) (layer "F.Cu") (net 6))
 (segment (start 78.441471 65.61) (end 76.375 65.61) (width 0.2) (layer "F.Cu") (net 6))
 (segment (start 82.135 66.77) (end 82.12 66.755) (width 0.2) (layer "F.Cu") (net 6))
 (segment (start 83.4445 66.77) (end 82.135 66.77) (width 0.2) (layer "F.Cu") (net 6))
 (segment (start 79.660396 65.709998) (end 79.555394 65.815) (width 0.2) (layer "F.Cu") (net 6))
 (via (at 79.660396 65.709998) (size 0.6) (drill 0.3) (layers "F.Cu" "B.Cu") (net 6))
 (via (at 82.12 66.755) (size 0.6) (drill 0.3) (layers "F.Cu" "B.Cu") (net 6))
 (segment (start 79.660396 65.709998) (end 81.074998 65.709998) (width 0.2) (layer "B.Cu") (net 6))
 (segment (start 79.660396 65.709998) (end 79.505002 65.709998) (width 0.2) (layer "B.Cu") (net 6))
 (segment (start 79.505002 65.709998) (end 79.105 66.11) (width 0.2) (layer "B.Cu") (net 6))
 (segment (start 81.074998 65.709998) (end 82.12 66.755) (width 0.2) (layer "B.Cu") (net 6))
 (segment (start 79.105 66.11) (end 76.375 66.11) (width 0.2) (layer "B.Cu") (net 6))
 (segment (start 83.635 68.365) (end 83.757 68.487) (width 0.2) (layer "F.Cu") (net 13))
 (segment (start 82.61 68.365) (end 83.635 68.365) (width 0.2) (layer "F.Cu") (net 13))
 (via (at 82.61 68.365) (size 0.6) (drill 0.3) (layers "F.Cu" "B.Cu") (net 13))
 (segment (start 82.46 68.405) (end 82.57 68.405) (width 0.2) (layer "B.Cu") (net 13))
 (segment (start 76.375 66.61) (end 78.325 66.61) (width 0.2) (layer "B.Cu") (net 13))
 (segment (start 82.57 68.405) (end 82.61 68.365) (width 0.2) (layer "B.Cu") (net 13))
 (segment (start 78.325 66.61) (end 80.12 68.405) (width 0.2) (layer "B.Cu") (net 13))
 (segment (start 80.12 68.405) (end 82.46 68.405) (width 0.2) (layer "B.Cu") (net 13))
 (segment (start 79.58 66.43) (end 79.58 66.365) (width 0.2) (layer "F.Cu") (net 7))
 (segment (start 83.4445 64.87) (end 82.145 64.87) (width 0.2) (layer "F.Cu") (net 7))
 (segment (start 82.145 64.87) (end 82.06 64.955) (width 0.2) (layer "F.Cu") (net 7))
 (segment (start 78.325 66.11) (end 76.375 66.11) (width 0.2) (layer "F.Cu") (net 7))
 (segment (start 79.58 66.365) (end 78.58 66.365) (width 0.2) (layer "F.Cu") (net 7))
 (segment (start 78.58 66.365) (end 78.325 66.11) (width 0.2) (layer "F.Cu") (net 7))
 (segment (start 79.66 66.51) (end 79.58 66.43) (width 0.2) (layer "F.Cu") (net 7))
 (via (at 82.06 64.955) (size 0.6) (drill 0.3) (layers "F.Cu" "B.Cu") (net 7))
 (via (at 79.66 66.51) (size 0.6) (drill 0.3) (layers "F.Cu" "B.Cu") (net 7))
 (segment (start 81.91 65.105) (end 82.06 64.955) (width 0.2) (layer "B.Cu") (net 7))
 (segment (start 82.368529 67.355) (end 82.72 67.003529) (width 0.2) (layer "B.Cu") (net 7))
 (segment (start 78.911865 65.61) (end 79.416865 65.105) (width 0.2) (layer "B.Cu") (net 7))
 (segment (start 76.375 65.61) (end 78.911865 65.61) (width 0.2) (layer "B.Cu") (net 7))
 (segment (start 82.72 65.615) (end 82.06 64.955) (width 0.2) (layer "B.Cu") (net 7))
 (segment (start 82.72 67.003529) (end 82.72 65.615) (width 0.2) (layer "B.Cu") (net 7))
 (segment (start 80.505 67.355) (end 82.368529 67.355) (width 0.2) (layer "B.Cu") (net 7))
 (segment (start 79.66 66.51) (end 80.505 67.355) (width 0.2) (layer "B.Cu") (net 7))
 (segment (start 79.416865 65.105) (end 81.91 65.105) (width 0.2) (layer "B.Cu") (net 7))
 (segment (start 90.185 79.21) (end 90.965 79.99) (width 0.2) (layer "F.Cu") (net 24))
 (segment (start 75.23 78.77) (end 79.99 78.77) (width 0.2) (layer "F.Cu") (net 24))
 (segment (start 84.64 82.17) (end 84.64 81.285001) (width 0.2) (layer "F.Cu") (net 24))
 (segment (start 84.114999 80.76) (end 83.4525 80.76) (width 0.2) (layer "F.Cu") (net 24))
 (segment (start 89.41 78.435) (end 90.185 79.21) (width 0.2) (layer "F.Cu") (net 24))
 (segment (start 90.965 79.99) (end 90.965 83.355) (width 0.2) (layer "F.Cu") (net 24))
 (segment (start 90.735 83.355) (end 95.615 83.355) (width 0.2) (layer "F.Cu") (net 24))
 (segment (start 90.965 83.355) (end 90.735 83.355) (width 0.2) (layer "F.Cu") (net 24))
 (segment (start 84.64 81.285001) (end 84.114999 80.76) (width 0.2) (layer "F.Cu") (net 24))
 (segment (start 82.855 78.435) (end 89.41 78.435) (width 0.2) (layer "F.Cu") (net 24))
 (segment (start 79.99 78.77) (end 82.52 78.77) (width 0.2) (layer "F.Cu") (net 24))
 (segment (start 89.4275 83.355) (end 88.6525 82.58) (width 0.2) (layer "F.Cu") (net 24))
 (segment (start 85.07 82.6) (end 84.64 82.17) (width 0.2) (layer "F.Cu") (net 24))
 (segment (start 82.52 78.77) (end 82.855 78.435) (width 0.2) (layer "F.Cu") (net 24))
 (segment (start 95.615 83.355) (end 96.91 84.65) (width 0.2) (layer "F.Cu") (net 24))
 (segment (start 90.735 83.355) (end 89.4275 83.355) (width 0.2) (layer "F.Cu") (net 24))
 (segment (start 88.6525 82.58) (end 88.6325 82.6) (width 0.2) (layer "F.Cu") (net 24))
 (segment (start 88.6325 82.6) (end 85.07 82.6) (width 0.2) (layer "F.Cu") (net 24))
 (segment (start 90.245 80.9) (end 90.245 82.5625) (width 0.2) (layer "F.Cu") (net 21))
 (segment (start 90.245 82.5625) (end 90.2275 82.58) (width 0.2) (layer "F.Cu") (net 21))
 (segment (start 85.7275 79.81) (end 87.19 79.81) (width 0.2) (layer "F.Cu") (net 23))
 (via (at 87.19 79.81) (size 0.6) (drill 0.3) (layers "F.Cu" "B.Cu") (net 23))
 (segment (start 98.06 79) (end 98.06 80.96) (width 0.2) (layer "B.Cu") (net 23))
 (segment (start 98.06 80.96) (end 96.91 82.11) (width 0.2) (layer "B.Cu") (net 23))
 (segment (start 88.58 78.42) (end 97.48 78.42) (width 0.2) (layer "B.Cu") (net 23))
 (segment (start 97.48 78.42) (end 98.06 79) (width 0.2) (layer "B.Cu") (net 23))
 (segment (start 87.19 79.81) (end 88.58 78.42) (width 0.2) (layer "B.Cu") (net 23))
 (segment (start 87.23 81.71) (end 87.24 81.72) (width 0.2) (layer "F.Cu") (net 22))
 (segment (start 85.7275 81.71) (end 87.23 81.71) (width 0.2) (layer "F.Cu") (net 22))
 (via (at 87.24 81.72) (size 0.6) (drill 0.3) (layers "F.Cu" "B.Cu") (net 22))
 (segment (start 94.76 81.72) (end 96.91 79.57) (width 0.2) (layer "B.Cu") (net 22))
 (segment (start 87.24 81.72) (end 94.76 81.72) (width 0.2) (layer "B.Cu") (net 22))
 (segment (start 79.79 81.37) (end 79.84 81.42) (width 0.2) (layer "F.Cu") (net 20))
 (segment (start 88.595 79.25) (end 88.635 79.21) (width 0.2) (layer "F.Cu") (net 20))
 (segment (start 79.84 81.42) (end 80.03 81.42) (width 0.2) (layer "F.Cu") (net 20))
 (segment (start 88.595 80.9) (end 88.595 79.25) (width 0.2) (layer "F.Cu") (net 20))
 (segment (start 75.23 81.37) (end 79.79 81.37) (width 0.2) (layer "F.Cu") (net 20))
 (via (at 80.03 81.42) (size 0.6) (drill 0.3) (layers "F.Cu" "B.Cu") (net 20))
 (segment (start 80.33 81.42) (end 84.72 77.03) (width 0.2) (layer "B.Cu") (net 20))
 (segment (start 84.72 77.03) (end 96.91 77.03) (width 0.2) (layer "B.Cu") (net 20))
 (segment (start 80.03 81.42) (end 80.33 81.42) (width 0.2) (layer "B.Cu") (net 20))
 (segment (start 83.4425 79.8) (end 79.2 79.8) (width 0.2) (layer "F.Cu") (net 26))
 (segment (start 79.2 79.8) (end 78.93 80.07) (width 0.2) (layer "F.Cu") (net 26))
 (segment (start 83.4525 79.81) (end 83.4425 79.8) (width 0.2) (layer "F.Cu") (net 26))
 (segment (start 78.93 80.07) (end 75.23 80.07) (width 0.2) (layer "F.Cu") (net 26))
 (segment (start 80.178529 80.72) (end 75.23 80.72) (width 0.2) (layer "F.Cu") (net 25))
 (segment (start 83.4525 81.71) (end 81.168529 81.71) (width 0.2) (layer "F.Cu") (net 25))
 (segment (start 81.168529 81.71) (end 80.178529 80.72) (width 0.2) (layer "F.Cu") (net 25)))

